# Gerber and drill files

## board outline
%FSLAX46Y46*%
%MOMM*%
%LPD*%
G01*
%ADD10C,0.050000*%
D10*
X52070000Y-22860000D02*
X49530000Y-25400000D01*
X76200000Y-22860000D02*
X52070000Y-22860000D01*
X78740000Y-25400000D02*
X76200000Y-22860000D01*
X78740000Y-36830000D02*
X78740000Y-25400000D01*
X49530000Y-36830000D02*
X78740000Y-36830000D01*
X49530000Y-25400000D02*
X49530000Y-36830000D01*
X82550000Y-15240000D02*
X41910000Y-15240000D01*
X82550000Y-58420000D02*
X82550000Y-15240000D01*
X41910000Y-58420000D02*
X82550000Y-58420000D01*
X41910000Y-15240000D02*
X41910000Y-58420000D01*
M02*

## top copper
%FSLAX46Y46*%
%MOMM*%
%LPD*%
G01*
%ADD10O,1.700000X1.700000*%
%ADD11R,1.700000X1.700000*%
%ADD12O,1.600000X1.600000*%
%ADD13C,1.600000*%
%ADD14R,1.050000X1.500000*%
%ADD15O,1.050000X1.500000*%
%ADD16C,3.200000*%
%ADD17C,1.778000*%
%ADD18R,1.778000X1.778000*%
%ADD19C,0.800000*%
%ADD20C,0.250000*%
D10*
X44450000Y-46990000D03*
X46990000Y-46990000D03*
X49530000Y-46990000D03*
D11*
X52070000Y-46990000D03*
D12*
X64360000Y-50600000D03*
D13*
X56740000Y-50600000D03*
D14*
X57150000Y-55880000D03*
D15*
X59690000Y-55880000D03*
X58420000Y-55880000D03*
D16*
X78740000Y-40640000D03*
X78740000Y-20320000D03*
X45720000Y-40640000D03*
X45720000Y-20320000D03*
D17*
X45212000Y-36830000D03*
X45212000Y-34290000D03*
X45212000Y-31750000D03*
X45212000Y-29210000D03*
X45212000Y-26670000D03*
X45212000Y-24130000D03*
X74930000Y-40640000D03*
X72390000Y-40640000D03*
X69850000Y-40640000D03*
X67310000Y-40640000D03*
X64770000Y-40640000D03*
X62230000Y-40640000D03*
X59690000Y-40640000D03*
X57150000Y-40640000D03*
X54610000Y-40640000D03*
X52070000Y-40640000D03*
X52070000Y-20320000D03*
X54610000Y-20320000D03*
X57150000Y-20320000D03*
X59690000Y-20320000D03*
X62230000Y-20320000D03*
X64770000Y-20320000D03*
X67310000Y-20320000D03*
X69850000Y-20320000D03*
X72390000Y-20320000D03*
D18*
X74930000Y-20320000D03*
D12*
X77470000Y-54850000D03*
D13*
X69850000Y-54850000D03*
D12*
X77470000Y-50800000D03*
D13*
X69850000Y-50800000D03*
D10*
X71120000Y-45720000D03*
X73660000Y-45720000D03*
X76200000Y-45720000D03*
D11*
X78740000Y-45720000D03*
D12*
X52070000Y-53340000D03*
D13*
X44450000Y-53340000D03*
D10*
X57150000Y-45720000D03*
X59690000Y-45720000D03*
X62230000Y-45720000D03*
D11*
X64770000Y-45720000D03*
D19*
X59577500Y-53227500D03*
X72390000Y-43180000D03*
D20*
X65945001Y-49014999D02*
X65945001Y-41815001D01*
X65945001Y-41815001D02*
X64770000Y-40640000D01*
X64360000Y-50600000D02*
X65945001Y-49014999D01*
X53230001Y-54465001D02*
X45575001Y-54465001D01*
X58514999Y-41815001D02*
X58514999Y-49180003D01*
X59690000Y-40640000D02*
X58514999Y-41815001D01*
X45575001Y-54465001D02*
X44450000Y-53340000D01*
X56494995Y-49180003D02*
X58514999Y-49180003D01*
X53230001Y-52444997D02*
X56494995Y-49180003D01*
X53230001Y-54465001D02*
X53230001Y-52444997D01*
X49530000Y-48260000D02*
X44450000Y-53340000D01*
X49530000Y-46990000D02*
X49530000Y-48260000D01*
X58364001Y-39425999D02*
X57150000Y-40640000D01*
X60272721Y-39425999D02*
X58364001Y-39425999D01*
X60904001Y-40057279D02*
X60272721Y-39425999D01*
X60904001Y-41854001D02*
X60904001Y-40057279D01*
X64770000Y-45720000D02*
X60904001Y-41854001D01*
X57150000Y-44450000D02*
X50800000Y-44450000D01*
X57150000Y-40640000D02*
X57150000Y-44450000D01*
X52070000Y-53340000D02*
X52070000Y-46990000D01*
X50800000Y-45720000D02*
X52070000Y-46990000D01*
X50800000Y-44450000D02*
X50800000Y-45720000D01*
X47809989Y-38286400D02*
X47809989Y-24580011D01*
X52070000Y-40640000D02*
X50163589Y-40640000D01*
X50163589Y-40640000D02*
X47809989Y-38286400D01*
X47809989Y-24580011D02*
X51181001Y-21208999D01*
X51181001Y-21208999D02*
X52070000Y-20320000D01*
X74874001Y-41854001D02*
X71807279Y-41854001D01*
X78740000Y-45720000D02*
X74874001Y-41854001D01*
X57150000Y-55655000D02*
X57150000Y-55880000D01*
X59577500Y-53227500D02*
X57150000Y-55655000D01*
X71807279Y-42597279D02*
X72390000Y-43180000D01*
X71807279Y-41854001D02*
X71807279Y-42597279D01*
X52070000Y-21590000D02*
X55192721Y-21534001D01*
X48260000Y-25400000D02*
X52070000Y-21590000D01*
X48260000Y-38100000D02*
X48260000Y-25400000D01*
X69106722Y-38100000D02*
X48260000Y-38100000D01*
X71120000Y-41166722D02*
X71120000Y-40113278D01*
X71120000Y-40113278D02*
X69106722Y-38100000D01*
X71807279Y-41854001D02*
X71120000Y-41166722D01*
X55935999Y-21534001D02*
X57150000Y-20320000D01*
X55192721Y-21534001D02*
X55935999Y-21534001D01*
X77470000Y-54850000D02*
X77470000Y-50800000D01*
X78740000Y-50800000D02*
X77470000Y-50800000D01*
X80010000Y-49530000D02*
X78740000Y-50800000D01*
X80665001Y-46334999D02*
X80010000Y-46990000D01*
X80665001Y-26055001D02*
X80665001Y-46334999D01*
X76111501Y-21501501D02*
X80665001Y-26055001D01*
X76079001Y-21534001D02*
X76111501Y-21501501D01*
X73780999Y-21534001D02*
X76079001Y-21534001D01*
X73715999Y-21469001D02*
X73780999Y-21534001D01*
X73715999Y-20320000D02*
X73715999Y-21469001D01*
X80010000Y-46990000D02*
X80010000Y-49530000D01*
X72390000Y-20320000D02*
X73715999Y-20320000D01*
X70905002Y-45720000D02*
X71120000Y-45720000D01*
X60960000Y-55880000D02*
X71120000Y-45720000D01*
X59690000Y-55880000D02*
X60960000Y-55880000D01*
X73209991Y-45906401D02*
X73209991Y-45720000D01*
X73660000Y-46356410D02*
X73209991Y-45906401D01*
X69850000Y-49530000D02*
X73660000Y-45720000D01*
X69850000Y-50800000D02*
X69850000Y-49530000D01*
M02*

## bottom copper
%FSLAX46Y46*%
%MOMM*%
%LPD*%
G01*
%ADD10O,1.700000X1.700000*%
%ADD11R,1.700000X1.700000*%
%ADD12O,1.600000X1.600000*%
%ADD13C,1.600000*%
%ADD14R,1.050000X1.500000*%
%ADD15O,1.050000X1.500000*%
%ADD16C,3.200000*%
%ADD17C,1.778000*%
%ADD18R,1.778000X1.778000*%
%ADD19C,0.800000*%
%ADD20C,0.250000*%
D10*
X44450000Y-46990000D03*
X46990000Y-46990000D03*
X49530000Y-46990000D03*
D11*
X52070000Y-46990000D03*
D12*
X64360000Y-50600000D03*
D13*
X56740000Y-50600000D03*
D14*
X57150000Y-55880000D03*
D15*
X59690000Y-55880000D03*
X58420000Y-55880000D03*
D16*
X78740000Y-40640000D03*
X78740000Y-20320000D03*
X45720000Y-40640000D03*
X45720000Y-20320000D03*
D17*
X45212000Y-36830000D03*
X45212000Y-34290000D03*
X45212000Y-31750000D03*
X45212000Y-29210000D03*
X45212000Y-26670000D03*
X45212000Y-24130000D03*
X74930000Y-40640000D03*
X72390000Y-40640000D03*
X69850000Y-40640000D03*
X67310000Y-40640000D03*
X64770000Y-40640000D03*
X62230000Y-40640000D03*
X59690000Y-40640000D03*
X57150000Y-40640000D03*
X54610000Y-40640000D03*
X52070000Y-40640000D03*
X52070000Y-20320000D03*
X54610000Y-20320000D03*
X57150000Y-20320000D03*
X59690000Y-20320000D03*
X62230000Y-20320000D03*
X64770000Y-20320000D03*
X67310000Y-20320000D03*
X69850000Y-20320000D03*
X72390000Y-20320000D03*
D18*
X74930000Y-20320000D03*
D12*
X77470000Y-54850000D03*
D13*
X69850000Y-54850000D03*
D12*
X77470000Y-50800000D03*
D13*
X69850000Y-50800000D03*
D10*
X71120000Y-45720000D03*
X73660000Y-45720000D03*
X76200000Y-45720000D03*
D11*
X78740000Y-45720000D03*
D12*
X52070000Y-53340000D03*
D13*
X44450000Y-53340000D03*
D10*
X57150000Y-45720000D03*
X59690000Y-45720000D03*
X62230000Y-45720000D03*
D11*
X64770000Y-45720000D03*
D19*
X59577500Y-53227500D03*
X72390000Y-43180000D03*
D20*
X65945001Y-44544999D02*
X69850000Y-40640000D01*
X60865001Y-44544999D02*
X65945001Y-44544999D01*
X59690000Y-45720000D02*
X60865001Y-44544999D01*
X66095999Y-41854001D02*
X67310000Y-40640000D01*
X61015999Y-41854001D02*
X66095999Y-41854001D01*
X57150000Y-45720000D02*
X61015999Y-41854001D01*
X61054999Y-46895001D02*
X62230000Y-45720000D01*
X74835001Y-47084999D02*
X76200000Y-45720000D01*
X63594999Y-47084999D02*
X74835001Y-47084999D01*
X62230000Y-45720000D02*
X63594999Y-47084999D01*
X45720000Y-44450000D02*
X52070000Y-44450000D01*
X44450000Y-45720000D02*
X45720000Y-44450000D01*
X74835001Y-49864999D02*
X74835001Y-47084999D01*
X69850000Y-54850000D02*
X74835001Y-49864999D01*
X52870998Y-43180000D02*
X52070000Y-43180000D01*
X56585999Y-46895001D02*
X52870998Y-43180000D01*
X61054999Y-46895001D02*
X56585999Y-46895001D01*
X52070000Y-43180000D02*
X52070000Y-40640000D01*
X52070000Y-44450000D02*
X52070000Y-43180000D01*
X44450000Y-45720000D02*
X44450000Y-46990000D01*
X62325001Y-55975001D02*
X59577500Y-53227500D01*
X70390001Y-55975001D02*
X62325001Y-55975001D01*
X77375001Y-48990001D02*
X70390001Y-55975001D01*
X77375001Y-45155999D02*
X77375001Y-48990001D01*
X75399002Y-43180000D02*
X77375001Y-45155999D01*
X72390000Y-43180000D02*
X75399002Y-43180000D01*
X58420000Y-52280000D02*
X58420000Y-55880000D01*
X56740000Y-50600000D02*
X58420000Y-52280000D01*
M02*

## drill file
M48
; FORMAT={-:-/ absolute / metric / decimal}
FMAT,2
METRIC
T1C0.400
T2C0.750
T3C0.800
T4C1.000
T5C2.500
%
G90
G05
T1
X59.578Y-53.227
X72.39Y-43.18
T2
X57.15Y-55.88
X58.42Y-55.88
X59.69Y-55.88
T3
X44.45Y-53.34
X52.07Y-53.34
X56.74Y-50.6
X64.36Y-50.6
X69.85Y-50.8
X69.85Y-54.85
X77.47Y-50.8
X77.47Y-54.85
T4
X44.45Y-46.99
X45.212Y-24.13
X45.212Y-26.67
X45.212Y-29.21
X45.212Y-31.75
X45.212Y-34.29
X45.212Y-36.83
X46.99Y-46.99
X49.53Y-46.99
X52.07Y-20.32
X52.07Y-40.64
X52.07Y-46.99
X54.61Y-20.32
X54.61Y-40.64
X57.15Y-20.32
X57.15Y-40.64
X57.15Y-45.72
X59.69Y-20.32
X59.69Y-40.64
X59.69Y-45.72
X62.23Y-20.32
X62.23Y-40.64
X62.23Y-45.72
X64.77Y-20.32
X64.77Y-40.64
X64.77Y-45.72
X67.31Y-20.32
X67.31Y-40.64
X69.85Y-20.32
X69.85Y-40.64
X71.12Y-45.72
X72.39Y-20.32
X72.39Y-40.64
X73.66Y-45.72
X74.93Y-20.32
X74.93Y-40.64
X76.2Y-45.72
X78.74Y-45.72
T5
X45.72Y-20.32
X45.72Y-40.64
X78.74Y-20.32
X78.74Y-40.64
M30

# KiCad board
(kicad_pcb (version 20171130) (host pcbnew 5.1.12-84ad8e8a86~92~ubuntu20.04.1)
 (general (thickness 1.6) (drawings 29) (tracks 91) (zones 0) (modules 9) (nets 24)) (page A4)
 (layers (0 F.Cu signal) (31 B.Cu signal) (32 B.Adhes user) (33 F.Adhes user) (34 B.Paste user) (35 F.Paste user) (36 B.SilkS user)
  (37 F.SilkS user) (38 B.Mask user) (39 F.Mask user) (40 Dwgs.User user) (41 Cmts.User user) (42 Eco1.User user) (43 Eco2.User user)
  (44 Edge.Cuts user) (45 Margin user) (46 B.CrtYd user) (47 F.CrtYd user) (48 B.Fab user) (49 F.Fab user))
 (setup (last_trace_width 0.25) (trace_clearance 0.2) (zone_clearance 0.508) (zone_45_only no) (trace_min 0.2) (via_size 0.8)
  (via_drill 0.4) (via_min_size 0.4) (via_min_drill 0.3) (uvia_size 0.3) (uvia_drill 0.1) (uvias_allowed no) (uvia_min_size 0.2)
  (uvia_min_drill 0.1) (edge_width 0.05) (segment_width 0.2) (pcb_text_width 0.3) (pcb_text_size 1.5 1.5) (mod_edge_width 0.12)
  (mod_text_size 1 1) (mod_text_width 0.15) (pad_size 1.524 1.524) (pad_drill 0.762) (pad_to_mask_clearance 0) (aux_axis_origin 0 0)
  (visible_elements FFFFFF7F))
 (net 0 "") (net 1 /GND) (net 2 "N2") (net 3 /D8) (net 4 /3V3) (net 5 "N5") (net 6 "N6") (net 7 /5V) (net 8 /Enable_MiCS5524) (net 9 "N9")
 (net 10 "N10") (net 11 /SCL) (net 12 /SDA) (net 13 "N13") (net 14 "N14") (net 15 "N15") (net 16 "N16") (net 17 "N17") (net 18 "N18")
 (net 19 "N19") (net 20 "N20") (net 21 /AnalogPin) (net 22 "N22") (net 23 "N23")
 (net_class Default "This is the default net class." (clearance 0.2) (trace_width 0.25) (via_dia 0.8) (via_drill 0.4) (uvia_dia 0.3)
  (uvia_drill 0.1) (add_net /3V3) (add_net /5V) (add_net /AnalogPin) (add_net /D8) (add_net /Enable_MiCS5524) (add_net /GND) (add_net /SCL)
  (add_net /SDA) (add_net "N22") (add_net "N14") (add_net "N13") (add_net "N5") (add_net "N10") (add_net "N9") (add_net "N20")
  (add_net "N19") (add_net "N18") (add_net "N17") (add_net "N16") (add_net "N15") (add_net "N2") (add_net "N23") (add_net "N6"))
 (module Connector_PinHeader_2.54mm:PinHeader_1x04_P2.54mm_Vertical (layer F.Cu) (at 52.07 46.99 270)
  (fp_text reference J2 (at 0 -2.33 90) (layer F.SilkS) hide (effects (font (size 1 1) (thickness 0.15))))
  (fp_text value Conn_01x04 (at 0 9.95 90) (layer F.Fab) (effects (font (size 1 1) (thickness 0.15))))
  (pad 4 thru_hole oval (at 0 7.62 270) (size 1.7 1.7) (drill 1) (layers *.Cu *.Mask) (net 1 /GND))
  (pad 3 thru_hole oval (at 0 5.08 270) (size 1.7 1.7) (drill 1) (layers *.Cu *.Mask) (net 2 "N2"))
  (pad 2 thru_hole oval (at 0 2.54 270) (size 1.7 1.7) (drill 1) (layers *.Cu *.Mask) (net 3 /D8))
  (pad 1 thru_hole rect (at 0 0 270) (size 1.7 1.7) (drill 1) (layers *.Cu *.Mask) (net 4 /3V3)))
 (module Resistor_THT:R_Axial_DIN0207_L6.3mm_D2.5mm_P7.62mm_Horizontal (layer F.Cu) (at 56.74 50.6)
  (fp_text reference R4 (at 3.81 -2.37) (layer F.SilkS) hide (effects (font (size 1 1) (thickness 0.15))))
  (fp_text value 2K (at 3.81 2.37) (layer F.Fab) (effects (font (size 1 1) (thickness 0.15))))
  (pad 2 thru_hole oval (at 7.62 0) (size 1.6 1.6) (drill 0.8) (layers *.Cu *.Mask) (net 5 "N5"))
  (pad 1 thru_hole circle (at 0 0) (size 1.6 1.6) (drill 0.8) (layers *.Cu *.Mask) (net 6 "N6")))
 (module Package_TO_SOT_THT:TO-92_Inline (layer F.Cu) (at 57.15 55.88)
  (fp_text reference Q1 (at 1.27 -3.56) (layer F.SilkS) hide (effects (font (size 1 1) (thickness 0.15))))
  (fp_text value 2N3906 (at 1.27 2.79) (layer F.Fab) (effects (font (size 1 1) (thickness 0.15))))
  (pad 1 thru_hole rect (at 0 0) (size 1.05 1.5) (drill 0.75) (layers *.Cu *.Mask) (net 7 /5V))
  (pad 3 thru_hole oval (at 2.54 0) (size 1.05 1.5) (drill 0.75) (layers *.Cu *.Mask) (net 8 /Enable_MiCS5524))
  (pad 2 thru_hole oval (at 1.27 0) (size 1.05 1.5) (drill 0.75) (layers *.Cu *.Mask) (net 6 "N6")))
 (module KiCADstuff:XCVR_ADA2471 (layer F.Cu) (at 62.23 30.48 270)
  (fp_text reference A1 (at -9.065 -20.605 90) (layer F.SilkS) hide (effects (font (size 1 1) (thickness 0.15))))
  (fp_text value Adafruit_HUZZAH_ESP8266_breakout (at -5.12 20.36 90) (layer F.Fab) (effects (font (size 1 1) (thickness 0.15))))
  (pad S4 thru_hole circle (at 10.16 -16.51 270) (size 3.2 3.2) (drill 2.5) (layers *.Cu *.Mask))
  (pad S3 thru_hole circle (at -10.16 -16.51 270) (size 3.2 3.2) (drill 2.5) (layers *.Cu *.Mask))
  (pad S2 thru_hole circle (at 10.16 16.51 270) (size 3.2 3.2) (drill 2.5) (layers *.Cu *.Mask))
  (pad S1 thru_hole circle (at -10.16 16.51 270) (size 3.2 3.2) (drill 2.5) (layers *.Cu *.Mask))
  (pad 26 thru_hole circle (at 6.35 17.018 270) (size 1.778 1.778) (drill 1) (layers *.Cu *.Mask))
  (pad 25 thru_hole circle (at 3.81 17.018 270) (size 1.778 1.778) (drill 1) (layers *.Cu *.Mask))
  (pad 24 thru_hole circle (at 1.27 17.018 270) (size 1.778 1.778) (drill 1) (layers *.Cu *.Mask))
  (pad 23 thru_hole circle (at -1.27 17.018 270) (size 1.778 1.778) (drill 1) (layers *.Cu *.Mask))
  (pad 22 thru_hole circle (at -3.81 17.018 270) (size 1.778 1.778) (drill 1) (layers *.Cu *.Mask))
  (pad 21 thru_hole circle (at -6.35 17.018 270) (size 1.778 1.778) (drill 1) (layers *.Cu *.Mask))
  (pad 20 thru_hole circle (at 10.16 -12.7 270) (size 1.778 1.778) (drill 1) (layers *.Cu *.Mask) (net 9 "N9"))
  (pad 19 thru_hole circle (at 10.16 -10.16 270) (size 1.778 1.778) (drill 1) (layers *.Cu *.Mask) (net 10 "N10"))
  (pad 18 thru_hole circle (at 10.16 -7.62 270) (size 1.778 1.778) (drill 1) (layers *.Cu *.Mask) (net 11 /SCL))
  (pad 17 thru_hole circle (at 10.16 -5.08 270) (size 1.778 1.778) (drill 1) (layers *.Cu *.Mask) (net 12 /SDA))
  (pad 16 thru_hole circle (at 10.16 -2.54 270) (size 1.778 1.778) (drill 1) (layers *.Cu *.Mask) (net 5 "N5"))
  (pad 15 thru_hole circle (at 10.16 0 270) (size 1.778 1.778) (drill 1) (layers *.Cu *.Mask) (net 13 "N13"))
  (pad 14 thru_hole circle (at 10.16 2.54 270) (size 1.778 1.778) (drill 1) (layers *.Cu *.Mask) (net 3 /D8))
  (pad 13 thru_hole circle (at 10.16 5.08 270) (size 1.778 1.778) (drill 1) (layers *.Cu *.Mask) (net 4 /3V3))
  (pad 12 thru_hole circle (at 10.16 7.62 270) (size 1.778 1.778) (drill 1) (layers *.Cu *.Mask) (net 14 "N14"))
  (pad 11 thru_hole circle (at 10.16 10.16 270) (size 1.778 1.778) (drill 1) (layers *.Cu *.Mask) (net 1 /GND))
  (pad 10 thru_hole circle (at -10.16 10.16 270) (size 1.778 1.778) (drill 1) (layers *.Cu *.Mask) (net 1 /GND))
  (pad 9 thru_hole circle (at -10.16 7.62 270) (size 1.778 1.778) (drill 1) (layers *.Cu *.Mask) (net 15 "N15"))
  (pad 8 thru_hole circle (at -10.16 5.08 270) (size 1.778 1.778) (drill 1) (layers *.Cu *.Mask) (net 7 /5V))
  (pad 7 thru_hole circle (at -10.16 2.54 270) (size 1.778 1.778) (drill 1) (layers *.Cu *.Mask) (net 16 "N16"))
  (pad 6 thru_hole circle (at -10.16 0 270) (size 1.778 1.778) (drill 1) (layers *.Cu *.Mask) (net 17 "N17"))
  (pad 5 thru_hole circle (at -10.16 -2.54 270) (size 1.778 1.778) (drill 1) (layers *.Cu *.Mask) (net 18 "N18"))
  (pad 4 thru_hole circle (at -10.16 -5.08 270) (size 1.778 1.778) (drill 1) (layers *.Cu *.Mask) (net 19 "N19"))
  (pad 3 thru_hole circle (at -10.16 -7.62 270) (size 1.778 1.778) (drill 1) (layers *.Cu *.Mask) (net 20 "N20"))
  (pad 2 thru_hole circle (at -10.16 -10.16 270) (size 1.778 1.778) (drill 1) (layers *.Cu *.Mask) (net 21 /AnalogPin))
  (pad 1 thru_hole rect (at -10.16 -12.7 270) (size 1.778 1.778) (drill 1) (layers *.Cu *.Mask) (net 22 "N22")))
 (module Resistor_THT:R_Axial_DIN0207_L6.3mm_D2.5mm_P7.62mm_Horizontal (layer F.Cu) (at 69.85 54.85)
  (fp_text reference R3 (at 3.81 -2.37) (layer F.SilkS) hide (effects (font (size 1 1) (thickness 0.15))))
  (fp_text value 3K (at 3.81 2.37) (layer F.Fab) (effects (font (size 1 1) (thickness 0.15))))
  (pad 2 thru_hole oval (at 7.62 0) (size 1.6 1.6) (drill 0.8) (layers *.Cu *.Mask) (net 21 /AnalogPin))
  (pad 1 thru_hole circle (at 0 0) (size 1.6 1.6) (drill 0.8) (layers *.Cu *.Mask) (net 1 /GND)))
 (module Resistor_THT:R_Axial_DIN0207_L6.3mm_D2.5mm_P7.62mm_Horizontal (layer F.Cu) (at 69.85 50.8)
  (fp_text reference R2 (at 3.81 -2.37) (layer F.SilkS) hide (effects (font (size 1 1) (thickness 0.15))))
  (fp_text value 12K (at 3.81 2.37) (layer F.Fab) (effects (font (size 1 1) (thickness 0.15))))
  (pad 2 thru_hole oval (at 7.62 0) (size 1.6 1.6) (drill 0.8) (layers *.Cu *.Mask) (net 21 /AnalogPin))
  (pad 1 thru_hole circle (at 0 0) (size 1.6 1.6) (drill 0.8) (layers *.Cu *.Mask) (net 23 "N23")))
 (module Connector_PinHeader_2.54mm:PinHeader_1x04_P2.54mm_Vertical (layer F.Cu) (at 78.74 45.72 270)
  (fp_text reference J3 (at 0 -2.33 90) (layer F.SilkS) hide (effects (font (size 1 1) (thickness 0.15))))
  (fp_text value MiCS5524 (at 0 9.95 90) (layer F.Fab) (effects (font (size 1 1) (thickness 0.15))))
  (pad 4 thru_hole oval (at 0 7.62 270) (size 1.7 1.7) (drill 1) (layers *.Cu *.Mask) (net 8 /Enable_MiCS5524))
  (pad 3 thru_hole oval (at 0 5.08 270) (size 1.7 1.7) (drill 1) (layers *.Cu *.Mask) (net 23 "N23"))
  (pad 2 thru_hole oval (at 0 2.54 270) (size 1.7 1.7) (drill 1) (layers *.Cu *.Mask) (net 1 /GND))
  (pad 1 thru_hole rect (at 0 0 270) (size 1.7 1.7) (drill 1) (layers *.Cu *.Mask) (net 7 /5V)))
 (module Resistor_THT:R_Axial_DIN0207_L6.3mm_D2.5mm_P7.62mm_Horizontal (layer F.Cu) (at 44.45 53.34)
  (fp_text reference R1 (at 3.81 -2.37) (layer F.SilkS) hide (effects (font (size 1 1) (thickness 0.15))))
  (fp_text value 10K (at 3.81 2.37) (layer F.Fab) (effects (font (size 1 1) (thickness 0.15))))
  (pad 2 thru_hole oval (at 7.62 0) (size 1.6 1.6) (drill 0.8) (layers *.Cu *.Mask) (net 4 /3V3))
  (pad 1 thru_hole circle (at 0 0) (size 1.6 1.6) (drill 0.8) (layers *.Cu *.Mask) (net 3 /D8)))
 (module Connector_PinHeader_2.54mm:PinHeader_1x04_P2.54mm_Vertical (layer F.Cu) (at 64.77 45.72 270)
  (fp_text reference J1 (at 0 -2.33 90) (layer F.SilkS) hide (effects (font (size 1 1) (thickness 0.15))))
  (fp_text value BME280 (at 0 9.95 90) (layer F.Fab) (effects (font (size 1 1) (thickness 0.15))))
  (pad 4 thru_hole oval (at 0 7.62 270) (size 1.7 1.7) (drill 1) (layers *.Cu *.Mask) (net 12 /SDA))
  (pad 3 thru_hole oval (at 0 5.08 270) (size 1.7 1.7) (drill 1) (layers *.Cu *.Mask) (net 11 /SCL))
  (pad 2 thru_hole oval (at 0 2.54 270) (size 1.7 1.7) (drill 1) (layers *.Cu *.Mask) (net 1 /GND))
  (pad 1 thru_hole rect (at 0 0 270) (size 1.7 1.7) (drill 1) (layers *.Cu *.Mask) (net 4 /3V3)))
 (gr_line (start 52.07 22.86) (end 49.53 25.4) (layer Edge.Cuts) (width 0.05))
 (gr_line (start 76.2 22.86) (end 52.07 22.86) (layer Edge.Cuts) (width 0.05))
 (gr_line (start 78.74 25.4) (end 76.2 22.86) (layer Edge.Cuts) (width 0.05))
 (gr_line (start 78.74 36.83) (end 78.74 25.4) (layer Edge.Cuts) (width 0.05))
 (gr_line (start 49.53 36.83) (end 78.74 36.83) (layer Edge.Cuts) (width 0.05))
 (gr_line (start 49.53 25.4) (end 49.53 36.83) (layer Edge.Cuts) (width 0.05))
 (gr_line (start 82.55 15.24) (end 41.91 15.24) (layer Edge.Cuts) (width 0.05))
 (gr_line (start 82.55 58.42) (end 82.55 15.24) (layer Edge.Cuts) (width 0.05))
 (gr_line (start 41.91 58.42) (end 82.55 58.42) (layer Edge.Cuts) (width 0.05))
 (gr_line (start 41.91 15.24) (end 41.91 58.42) (layer Edge.Cuts) (width 0.05))
 (segment (start 65.945001 44.544999) (end 69.85 40.64) (width 0.25) (layer B.Cu) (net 11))
 (segment (start 60.865001 44.544999) (end 65.945001 44.544999) (width 0.25) (layer B.Cu) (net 11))
 (segment (start 59.69 45.72) (end 60.865001 44.544999) (width 0.25) (layer B.Cu) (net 11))
 (segment (start 66.095999 41.854001) (end 67.31 40.64) (width 0.25) (layer B.Cu) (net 12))
 (segment (start 61.015999 41.854001) (end 66.095999 41.854001) (width 0.25) (layer B.Cu) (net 12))
 (segment (start 57.15 45.72) (end 61.015999 41.854001) (width 0.25) (layer B.Cu) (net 12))
 (segment (start 65.945001 49.014999) (end 65.945001 41.815001) (width 0.25) (layer F.Cu) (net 5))
 (segment (start 65.945001 41.815001) (end 64.77 40.64) (width 0.25) (layer F.Cu) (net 5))
 (segment (start 64.36 50.6) (end 65.945001 49.014999) (width 0.25) (layer F.Cu) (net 5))
 (segment (start 53.230001 54.465001) (end 45.575001 54.465001) (width 0.25) (layer F.Cu) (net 3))
 (segment (start 58.514999 41.815001) (end 58.514999 49.180003) (width 0.25) (layer F.Cu) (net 3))
 (segment (start 59.69 40.64) (end 58.514999 41.815001) (width 0.25) (layer F.Cu) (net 3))
 (segment (start 45.575001 54.465001) (end 44.45 53.34) (width 0.25) (layer F.Cu) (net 3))
 (segment (start 56.494995 49.180003) (end 58.514999 49.180003) (width 0.25) (layer F.Cu) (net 3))
 (segment (start 53.230001 52.444997) (end 56.494995 49.180003) (width 0.25) (layer F.Cu) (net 3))
 (segment (start 53.230001 54.465001) (end 53.230001 52.444997) (width 0.25) (layer F.Cu) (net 3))
 (segment (start 49.53 48.26) (end 44.45 53.34) (width 0.25) (layer F.Cu) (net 3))
 (segment (start 49.53 46.99) (end 49.53 48.26) (width 0.25) (layer F.Cu) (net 3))
 (segment (start 58.364001 39.425999) (end 57.15 40.64) (width 0.25) (layer F.Cu) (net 4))
 (segment (start 60.272721 39.425999) (end 58.364001 39.425999) (width 0.25) (layer F.Cu) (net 4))
 (segment (start 60.904001 40.057279) (end 60.272721 39.425999) (width 0.25) (layer F.Cu) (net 4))
 (segment (start 60.904001 41.854001) (end 60.904001 40.057279) (width 0.25) (layer F.Cu) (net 4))
 (segment (start 64.77 45.72) (end 60.904001 41.854001) (width 0.25) (layer F.Cu) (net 4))
 (segment (start 57.15 44.45) (end 50.8 44.45) (width 0.25) (layer F.Cu) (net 4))
 (segment (start 57.15 40.64) (end 57.15 44.45) (width 0.25) (layer F.Cu) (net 4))
 (segment (start 52.07 53.34) (end 52.07 46.99) (width 0.25) (layer F.Cu) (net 4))
 (segment (start 50.8 45.72) (end 52.07 46.99) (width 0.25) (layer F.Cu) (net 4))
 (segment (start 50.8 44.45) (end 50.8 45.72) (width 0.25) (layer F.Cu) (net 4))
 (segment (start 61.054999 46.895001) (end 62.23 45.72) (width 0.25) (layer B.Cu) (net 1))
 (segment (start 74.835001 47.084999) (end 76.2 45.72) (width 0.25) (layer B.Cu) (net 1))
 (segment (start 63.594999 47.084999) (end 74.835001 47.084999) (width 0.25) (layer B.Cu) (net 1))
 (segment (start 62.23 45.72) (end 63.594999 47.084999) (width 0.25) (layer B.Cu) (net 1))
 (segment (start 45.72 44.45) (end 52.07 44.45) (width 0.25) (layer B.Cu) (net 1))
 (segment (start 44.45 45.72) (end 45.72 44.45) (width 0.25) (layer B.Cu) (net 1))
 (segment (start 74.835001 49.864999) (end 74.835001 47.084999) (width 0.25) (layer B.Cu) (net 1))
 (segment (start 69.85 54.85) (end 74.835001 49.864999) (width 0.25) (layer B.Cu) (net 1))
 (segment (start 52.870998 43.18) (end 52.07 43.18) (width 0.25) (layer B.Cu) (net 1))
 (segment (start 56.585999 46.895001) (end 52.870998 43.18) (width 0.25) (layer B.Cu) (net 1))
 (segment (start 61.054999 46.895001) (end 56.585999 46.895001) (width 0.25) (layer B.Cu) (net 1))
 (segment (start 52.07 43.18) (end 52.07 40.64) (width 0.25) (layer B.Cu) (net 1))
 (segment (start 52.07 44.45) (end 52.07 43.18) (width 0.25) (layer B.Cu) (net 1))
 (segment (start 44.45 45.72) (end 44.45 46.99) (width 0.25) (layer B.Cu) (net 1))
 (segment (start 47.809989 38.2864) (end 47.809989 24.580011) (width 0.25) (layer F.Cu) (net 1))
 (segment (start 52.07 40.64) (end 50.163589 40.64) (width 0.25) (layer F.Cu) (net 1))
 (segment (start 50.163589 40.64) (end 47.809989 38.2864) (width 0.25) (layer F.Cu) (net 1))
 (segment (start 47.809989 24.580011) (end 51.181001 21.208999) (width 0.25) (layer F.Cu) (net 1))
 (segment (start 51.181001 21.208999) (end 52.07 20.32) (width 0.25) (layer F.Cu) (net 1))
 (segment (start 74.874001 41.854001) (end 71.807279 41.854001) (width 0.25) (layer F.Cu) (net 7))
 (segment (start 78.74 45.72) (end 74.874001 41.854001) (width 0.25) (layer F.Cu) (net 7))
 (segment (start 57.15 55.655) (end 57.15 55.88) (width 0.25) (layer F.Cu) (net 7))
 (segment (start 59.5775 53.2275) (end 57.15 55.655) (width 0.25) (layer F.Cu) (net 7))
 (via (at 59.5775 53.2275) (size 0.8) (drill 0.4) (layers F.Cu B.Cu) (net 7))
 (via (at 72.39 43.18) (size 0.8) (drill 0.4) (layers F.Cu B.Cu) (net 7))
 (segment (start 71.807279 42.597279) (end 72.39 43.18) (width 0.25) (layer F.Cu) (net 7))
 (segment (start 71.807279 41.854001) (end 71.807279 42.597279) (width 0.25) (layer F.Cu) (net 7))
 (segment (start 62.325001 55.975001) (end 59.5775 53.2275) (width 0.25) (layer B.Cu) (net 7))
 (segment (start 70.390001 55.975001) (end 62.325001 55.975001) (width 0.25) (layer B.Cu) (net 7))
 (segment (start 77.375001 48.990001) (end 70.390001 55.975001) (width 0.25) (layer B.Cu) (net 7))
 (segment (start 77.375001 45.155999) (end 77.375001 48.990001) (width 0.25) (layer B.Cu) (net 7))
 (segment (start 75.399002 43.18) (end 77.375001 45.155999) (width 0.25) (layer B.Cu) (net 7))
 (segment (start 72.39 43.18) (end 75.399002 43.18) (width 0.25) (layer B.Cu) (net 7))
 (segment (start 52.07 21.59) (end 55.192721 21.534001) (width 0.25) (layer F.Cu) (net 7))
 (segment (start 48.26 25.4) (end 52.07 21.59) (width 0.25) (layer F.Cu) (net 7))
 (segment (start 48.26 38.1) (end 48.26 25.4) (width 0.25) (layer F.Cu) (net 7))
 (segment (start 69.106722 38.1) (end 48.26 38.1) (width 0.25) (layer F.Cu) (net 7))
 (segment (start 71.12 41.166722) (end 71.12 40.113278) (width 0.25) (layer F.Cu) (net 7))
 (segment (start 71.12 40.113278) (end 69.106722 38.1) (width 0.25) (layer F.Cu) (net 7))
 (segment (start 71.807279 41.854001) (end 71.12 41.166722) (width 0.25) (layer F.Cu) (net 7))
 (segment (start 55.935999 21.534001) (end 57.15 20.32) (width 0.25) (layer F.Cu) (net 7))
 (segment (start 55.192721 21.534001) (end 55.935999 21.534001) (width 0.25) (layer F.Cu) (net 7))
 (segment (start 77.47 54.85) (end 77.47 50.8) (width 0.25) (layer F.Cu) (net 21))
 (segment (start 78.74 50.8) (end 77.47 50.8) (width 0.25) (layer F.Cu) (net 21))
 (segment (start 80.01 49.53) (end 78.74 50.8) (width 0.25) (layer F.Cu) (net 21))
 (segment (start 80.665001 46.334999) (end 80.01 46.99) (width 0.25) (layer F.Cu) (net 21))
 (segment (start 80.665001 26.055001) (end 80.665001 46.334999) (width 0.25) (layer F.Cu) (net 21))
 (segment (start 76.111501 21.501501) (end 80.665001 26.055001) (width 0.25) (layer F.Cu) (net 21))
 (segment (start 76.079001 21.534001) (end 76.111501 21.501501) (width 0.25) (layer F.Cu) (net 21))
 (segment (start 73.780999 21.534001) (end 76.079001 21.534001) (width 0.25) (layer F.Cu) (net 21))
 (segment (start 73.715999 21.469001) (end 73.780999 21.534001) (width 0.25) (layer F.Cu) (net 21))
 (segment (start 73.715999 20.32) (end 73.715999 21.469001) (width 0.25) (layer F.Cu) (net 21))
 (segment (start 80.01 46.99) (end 80.01 49.53) (width 0.25) (layer F.Cu) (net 21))
 (segment (start 72.39 20.32) (end 73.715999 20.32) (width 0.25) (layer F.Cu) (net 21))
 (segment (start 70.905002 45.72) (end 71.12 45.72) (width 0.25) (layer F.Cu) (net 8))
 (segment (start 60.96 55.88) (end 71.12 45.72) (width 0.25) (layer F.Cu) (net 8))
 (segment (start 59.69 55.88) (end 60.96 55.88) (width 0.25) (layer F.Cu) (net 8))
 (segment (start 73.209991 45.906401) (end 73.209991 45.72) (width 0.25) (layer F.Cu) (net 23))
 (segment (start 73.66 46.35641) (end 73.209991 45.906401) (width 0.25) (layer F.Cu) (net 23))
 (segment (start 69.85 49.53) (end 73.66 45.72) (width 0.25) (layer F.Cu) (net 23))
 (segment (start 69.85 50.8) (end 69.85 49.53) (width 0.25) (layer F.Cu) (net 23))
 (segment (start 58.42 52.28) (end 58.42 55.88) (width 0.25) (layer B.Cu) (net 6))
 (segment (start 56.74 50.6) (end 58.42 52.28) (width 0.25) (layer B.Cu) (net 6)))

